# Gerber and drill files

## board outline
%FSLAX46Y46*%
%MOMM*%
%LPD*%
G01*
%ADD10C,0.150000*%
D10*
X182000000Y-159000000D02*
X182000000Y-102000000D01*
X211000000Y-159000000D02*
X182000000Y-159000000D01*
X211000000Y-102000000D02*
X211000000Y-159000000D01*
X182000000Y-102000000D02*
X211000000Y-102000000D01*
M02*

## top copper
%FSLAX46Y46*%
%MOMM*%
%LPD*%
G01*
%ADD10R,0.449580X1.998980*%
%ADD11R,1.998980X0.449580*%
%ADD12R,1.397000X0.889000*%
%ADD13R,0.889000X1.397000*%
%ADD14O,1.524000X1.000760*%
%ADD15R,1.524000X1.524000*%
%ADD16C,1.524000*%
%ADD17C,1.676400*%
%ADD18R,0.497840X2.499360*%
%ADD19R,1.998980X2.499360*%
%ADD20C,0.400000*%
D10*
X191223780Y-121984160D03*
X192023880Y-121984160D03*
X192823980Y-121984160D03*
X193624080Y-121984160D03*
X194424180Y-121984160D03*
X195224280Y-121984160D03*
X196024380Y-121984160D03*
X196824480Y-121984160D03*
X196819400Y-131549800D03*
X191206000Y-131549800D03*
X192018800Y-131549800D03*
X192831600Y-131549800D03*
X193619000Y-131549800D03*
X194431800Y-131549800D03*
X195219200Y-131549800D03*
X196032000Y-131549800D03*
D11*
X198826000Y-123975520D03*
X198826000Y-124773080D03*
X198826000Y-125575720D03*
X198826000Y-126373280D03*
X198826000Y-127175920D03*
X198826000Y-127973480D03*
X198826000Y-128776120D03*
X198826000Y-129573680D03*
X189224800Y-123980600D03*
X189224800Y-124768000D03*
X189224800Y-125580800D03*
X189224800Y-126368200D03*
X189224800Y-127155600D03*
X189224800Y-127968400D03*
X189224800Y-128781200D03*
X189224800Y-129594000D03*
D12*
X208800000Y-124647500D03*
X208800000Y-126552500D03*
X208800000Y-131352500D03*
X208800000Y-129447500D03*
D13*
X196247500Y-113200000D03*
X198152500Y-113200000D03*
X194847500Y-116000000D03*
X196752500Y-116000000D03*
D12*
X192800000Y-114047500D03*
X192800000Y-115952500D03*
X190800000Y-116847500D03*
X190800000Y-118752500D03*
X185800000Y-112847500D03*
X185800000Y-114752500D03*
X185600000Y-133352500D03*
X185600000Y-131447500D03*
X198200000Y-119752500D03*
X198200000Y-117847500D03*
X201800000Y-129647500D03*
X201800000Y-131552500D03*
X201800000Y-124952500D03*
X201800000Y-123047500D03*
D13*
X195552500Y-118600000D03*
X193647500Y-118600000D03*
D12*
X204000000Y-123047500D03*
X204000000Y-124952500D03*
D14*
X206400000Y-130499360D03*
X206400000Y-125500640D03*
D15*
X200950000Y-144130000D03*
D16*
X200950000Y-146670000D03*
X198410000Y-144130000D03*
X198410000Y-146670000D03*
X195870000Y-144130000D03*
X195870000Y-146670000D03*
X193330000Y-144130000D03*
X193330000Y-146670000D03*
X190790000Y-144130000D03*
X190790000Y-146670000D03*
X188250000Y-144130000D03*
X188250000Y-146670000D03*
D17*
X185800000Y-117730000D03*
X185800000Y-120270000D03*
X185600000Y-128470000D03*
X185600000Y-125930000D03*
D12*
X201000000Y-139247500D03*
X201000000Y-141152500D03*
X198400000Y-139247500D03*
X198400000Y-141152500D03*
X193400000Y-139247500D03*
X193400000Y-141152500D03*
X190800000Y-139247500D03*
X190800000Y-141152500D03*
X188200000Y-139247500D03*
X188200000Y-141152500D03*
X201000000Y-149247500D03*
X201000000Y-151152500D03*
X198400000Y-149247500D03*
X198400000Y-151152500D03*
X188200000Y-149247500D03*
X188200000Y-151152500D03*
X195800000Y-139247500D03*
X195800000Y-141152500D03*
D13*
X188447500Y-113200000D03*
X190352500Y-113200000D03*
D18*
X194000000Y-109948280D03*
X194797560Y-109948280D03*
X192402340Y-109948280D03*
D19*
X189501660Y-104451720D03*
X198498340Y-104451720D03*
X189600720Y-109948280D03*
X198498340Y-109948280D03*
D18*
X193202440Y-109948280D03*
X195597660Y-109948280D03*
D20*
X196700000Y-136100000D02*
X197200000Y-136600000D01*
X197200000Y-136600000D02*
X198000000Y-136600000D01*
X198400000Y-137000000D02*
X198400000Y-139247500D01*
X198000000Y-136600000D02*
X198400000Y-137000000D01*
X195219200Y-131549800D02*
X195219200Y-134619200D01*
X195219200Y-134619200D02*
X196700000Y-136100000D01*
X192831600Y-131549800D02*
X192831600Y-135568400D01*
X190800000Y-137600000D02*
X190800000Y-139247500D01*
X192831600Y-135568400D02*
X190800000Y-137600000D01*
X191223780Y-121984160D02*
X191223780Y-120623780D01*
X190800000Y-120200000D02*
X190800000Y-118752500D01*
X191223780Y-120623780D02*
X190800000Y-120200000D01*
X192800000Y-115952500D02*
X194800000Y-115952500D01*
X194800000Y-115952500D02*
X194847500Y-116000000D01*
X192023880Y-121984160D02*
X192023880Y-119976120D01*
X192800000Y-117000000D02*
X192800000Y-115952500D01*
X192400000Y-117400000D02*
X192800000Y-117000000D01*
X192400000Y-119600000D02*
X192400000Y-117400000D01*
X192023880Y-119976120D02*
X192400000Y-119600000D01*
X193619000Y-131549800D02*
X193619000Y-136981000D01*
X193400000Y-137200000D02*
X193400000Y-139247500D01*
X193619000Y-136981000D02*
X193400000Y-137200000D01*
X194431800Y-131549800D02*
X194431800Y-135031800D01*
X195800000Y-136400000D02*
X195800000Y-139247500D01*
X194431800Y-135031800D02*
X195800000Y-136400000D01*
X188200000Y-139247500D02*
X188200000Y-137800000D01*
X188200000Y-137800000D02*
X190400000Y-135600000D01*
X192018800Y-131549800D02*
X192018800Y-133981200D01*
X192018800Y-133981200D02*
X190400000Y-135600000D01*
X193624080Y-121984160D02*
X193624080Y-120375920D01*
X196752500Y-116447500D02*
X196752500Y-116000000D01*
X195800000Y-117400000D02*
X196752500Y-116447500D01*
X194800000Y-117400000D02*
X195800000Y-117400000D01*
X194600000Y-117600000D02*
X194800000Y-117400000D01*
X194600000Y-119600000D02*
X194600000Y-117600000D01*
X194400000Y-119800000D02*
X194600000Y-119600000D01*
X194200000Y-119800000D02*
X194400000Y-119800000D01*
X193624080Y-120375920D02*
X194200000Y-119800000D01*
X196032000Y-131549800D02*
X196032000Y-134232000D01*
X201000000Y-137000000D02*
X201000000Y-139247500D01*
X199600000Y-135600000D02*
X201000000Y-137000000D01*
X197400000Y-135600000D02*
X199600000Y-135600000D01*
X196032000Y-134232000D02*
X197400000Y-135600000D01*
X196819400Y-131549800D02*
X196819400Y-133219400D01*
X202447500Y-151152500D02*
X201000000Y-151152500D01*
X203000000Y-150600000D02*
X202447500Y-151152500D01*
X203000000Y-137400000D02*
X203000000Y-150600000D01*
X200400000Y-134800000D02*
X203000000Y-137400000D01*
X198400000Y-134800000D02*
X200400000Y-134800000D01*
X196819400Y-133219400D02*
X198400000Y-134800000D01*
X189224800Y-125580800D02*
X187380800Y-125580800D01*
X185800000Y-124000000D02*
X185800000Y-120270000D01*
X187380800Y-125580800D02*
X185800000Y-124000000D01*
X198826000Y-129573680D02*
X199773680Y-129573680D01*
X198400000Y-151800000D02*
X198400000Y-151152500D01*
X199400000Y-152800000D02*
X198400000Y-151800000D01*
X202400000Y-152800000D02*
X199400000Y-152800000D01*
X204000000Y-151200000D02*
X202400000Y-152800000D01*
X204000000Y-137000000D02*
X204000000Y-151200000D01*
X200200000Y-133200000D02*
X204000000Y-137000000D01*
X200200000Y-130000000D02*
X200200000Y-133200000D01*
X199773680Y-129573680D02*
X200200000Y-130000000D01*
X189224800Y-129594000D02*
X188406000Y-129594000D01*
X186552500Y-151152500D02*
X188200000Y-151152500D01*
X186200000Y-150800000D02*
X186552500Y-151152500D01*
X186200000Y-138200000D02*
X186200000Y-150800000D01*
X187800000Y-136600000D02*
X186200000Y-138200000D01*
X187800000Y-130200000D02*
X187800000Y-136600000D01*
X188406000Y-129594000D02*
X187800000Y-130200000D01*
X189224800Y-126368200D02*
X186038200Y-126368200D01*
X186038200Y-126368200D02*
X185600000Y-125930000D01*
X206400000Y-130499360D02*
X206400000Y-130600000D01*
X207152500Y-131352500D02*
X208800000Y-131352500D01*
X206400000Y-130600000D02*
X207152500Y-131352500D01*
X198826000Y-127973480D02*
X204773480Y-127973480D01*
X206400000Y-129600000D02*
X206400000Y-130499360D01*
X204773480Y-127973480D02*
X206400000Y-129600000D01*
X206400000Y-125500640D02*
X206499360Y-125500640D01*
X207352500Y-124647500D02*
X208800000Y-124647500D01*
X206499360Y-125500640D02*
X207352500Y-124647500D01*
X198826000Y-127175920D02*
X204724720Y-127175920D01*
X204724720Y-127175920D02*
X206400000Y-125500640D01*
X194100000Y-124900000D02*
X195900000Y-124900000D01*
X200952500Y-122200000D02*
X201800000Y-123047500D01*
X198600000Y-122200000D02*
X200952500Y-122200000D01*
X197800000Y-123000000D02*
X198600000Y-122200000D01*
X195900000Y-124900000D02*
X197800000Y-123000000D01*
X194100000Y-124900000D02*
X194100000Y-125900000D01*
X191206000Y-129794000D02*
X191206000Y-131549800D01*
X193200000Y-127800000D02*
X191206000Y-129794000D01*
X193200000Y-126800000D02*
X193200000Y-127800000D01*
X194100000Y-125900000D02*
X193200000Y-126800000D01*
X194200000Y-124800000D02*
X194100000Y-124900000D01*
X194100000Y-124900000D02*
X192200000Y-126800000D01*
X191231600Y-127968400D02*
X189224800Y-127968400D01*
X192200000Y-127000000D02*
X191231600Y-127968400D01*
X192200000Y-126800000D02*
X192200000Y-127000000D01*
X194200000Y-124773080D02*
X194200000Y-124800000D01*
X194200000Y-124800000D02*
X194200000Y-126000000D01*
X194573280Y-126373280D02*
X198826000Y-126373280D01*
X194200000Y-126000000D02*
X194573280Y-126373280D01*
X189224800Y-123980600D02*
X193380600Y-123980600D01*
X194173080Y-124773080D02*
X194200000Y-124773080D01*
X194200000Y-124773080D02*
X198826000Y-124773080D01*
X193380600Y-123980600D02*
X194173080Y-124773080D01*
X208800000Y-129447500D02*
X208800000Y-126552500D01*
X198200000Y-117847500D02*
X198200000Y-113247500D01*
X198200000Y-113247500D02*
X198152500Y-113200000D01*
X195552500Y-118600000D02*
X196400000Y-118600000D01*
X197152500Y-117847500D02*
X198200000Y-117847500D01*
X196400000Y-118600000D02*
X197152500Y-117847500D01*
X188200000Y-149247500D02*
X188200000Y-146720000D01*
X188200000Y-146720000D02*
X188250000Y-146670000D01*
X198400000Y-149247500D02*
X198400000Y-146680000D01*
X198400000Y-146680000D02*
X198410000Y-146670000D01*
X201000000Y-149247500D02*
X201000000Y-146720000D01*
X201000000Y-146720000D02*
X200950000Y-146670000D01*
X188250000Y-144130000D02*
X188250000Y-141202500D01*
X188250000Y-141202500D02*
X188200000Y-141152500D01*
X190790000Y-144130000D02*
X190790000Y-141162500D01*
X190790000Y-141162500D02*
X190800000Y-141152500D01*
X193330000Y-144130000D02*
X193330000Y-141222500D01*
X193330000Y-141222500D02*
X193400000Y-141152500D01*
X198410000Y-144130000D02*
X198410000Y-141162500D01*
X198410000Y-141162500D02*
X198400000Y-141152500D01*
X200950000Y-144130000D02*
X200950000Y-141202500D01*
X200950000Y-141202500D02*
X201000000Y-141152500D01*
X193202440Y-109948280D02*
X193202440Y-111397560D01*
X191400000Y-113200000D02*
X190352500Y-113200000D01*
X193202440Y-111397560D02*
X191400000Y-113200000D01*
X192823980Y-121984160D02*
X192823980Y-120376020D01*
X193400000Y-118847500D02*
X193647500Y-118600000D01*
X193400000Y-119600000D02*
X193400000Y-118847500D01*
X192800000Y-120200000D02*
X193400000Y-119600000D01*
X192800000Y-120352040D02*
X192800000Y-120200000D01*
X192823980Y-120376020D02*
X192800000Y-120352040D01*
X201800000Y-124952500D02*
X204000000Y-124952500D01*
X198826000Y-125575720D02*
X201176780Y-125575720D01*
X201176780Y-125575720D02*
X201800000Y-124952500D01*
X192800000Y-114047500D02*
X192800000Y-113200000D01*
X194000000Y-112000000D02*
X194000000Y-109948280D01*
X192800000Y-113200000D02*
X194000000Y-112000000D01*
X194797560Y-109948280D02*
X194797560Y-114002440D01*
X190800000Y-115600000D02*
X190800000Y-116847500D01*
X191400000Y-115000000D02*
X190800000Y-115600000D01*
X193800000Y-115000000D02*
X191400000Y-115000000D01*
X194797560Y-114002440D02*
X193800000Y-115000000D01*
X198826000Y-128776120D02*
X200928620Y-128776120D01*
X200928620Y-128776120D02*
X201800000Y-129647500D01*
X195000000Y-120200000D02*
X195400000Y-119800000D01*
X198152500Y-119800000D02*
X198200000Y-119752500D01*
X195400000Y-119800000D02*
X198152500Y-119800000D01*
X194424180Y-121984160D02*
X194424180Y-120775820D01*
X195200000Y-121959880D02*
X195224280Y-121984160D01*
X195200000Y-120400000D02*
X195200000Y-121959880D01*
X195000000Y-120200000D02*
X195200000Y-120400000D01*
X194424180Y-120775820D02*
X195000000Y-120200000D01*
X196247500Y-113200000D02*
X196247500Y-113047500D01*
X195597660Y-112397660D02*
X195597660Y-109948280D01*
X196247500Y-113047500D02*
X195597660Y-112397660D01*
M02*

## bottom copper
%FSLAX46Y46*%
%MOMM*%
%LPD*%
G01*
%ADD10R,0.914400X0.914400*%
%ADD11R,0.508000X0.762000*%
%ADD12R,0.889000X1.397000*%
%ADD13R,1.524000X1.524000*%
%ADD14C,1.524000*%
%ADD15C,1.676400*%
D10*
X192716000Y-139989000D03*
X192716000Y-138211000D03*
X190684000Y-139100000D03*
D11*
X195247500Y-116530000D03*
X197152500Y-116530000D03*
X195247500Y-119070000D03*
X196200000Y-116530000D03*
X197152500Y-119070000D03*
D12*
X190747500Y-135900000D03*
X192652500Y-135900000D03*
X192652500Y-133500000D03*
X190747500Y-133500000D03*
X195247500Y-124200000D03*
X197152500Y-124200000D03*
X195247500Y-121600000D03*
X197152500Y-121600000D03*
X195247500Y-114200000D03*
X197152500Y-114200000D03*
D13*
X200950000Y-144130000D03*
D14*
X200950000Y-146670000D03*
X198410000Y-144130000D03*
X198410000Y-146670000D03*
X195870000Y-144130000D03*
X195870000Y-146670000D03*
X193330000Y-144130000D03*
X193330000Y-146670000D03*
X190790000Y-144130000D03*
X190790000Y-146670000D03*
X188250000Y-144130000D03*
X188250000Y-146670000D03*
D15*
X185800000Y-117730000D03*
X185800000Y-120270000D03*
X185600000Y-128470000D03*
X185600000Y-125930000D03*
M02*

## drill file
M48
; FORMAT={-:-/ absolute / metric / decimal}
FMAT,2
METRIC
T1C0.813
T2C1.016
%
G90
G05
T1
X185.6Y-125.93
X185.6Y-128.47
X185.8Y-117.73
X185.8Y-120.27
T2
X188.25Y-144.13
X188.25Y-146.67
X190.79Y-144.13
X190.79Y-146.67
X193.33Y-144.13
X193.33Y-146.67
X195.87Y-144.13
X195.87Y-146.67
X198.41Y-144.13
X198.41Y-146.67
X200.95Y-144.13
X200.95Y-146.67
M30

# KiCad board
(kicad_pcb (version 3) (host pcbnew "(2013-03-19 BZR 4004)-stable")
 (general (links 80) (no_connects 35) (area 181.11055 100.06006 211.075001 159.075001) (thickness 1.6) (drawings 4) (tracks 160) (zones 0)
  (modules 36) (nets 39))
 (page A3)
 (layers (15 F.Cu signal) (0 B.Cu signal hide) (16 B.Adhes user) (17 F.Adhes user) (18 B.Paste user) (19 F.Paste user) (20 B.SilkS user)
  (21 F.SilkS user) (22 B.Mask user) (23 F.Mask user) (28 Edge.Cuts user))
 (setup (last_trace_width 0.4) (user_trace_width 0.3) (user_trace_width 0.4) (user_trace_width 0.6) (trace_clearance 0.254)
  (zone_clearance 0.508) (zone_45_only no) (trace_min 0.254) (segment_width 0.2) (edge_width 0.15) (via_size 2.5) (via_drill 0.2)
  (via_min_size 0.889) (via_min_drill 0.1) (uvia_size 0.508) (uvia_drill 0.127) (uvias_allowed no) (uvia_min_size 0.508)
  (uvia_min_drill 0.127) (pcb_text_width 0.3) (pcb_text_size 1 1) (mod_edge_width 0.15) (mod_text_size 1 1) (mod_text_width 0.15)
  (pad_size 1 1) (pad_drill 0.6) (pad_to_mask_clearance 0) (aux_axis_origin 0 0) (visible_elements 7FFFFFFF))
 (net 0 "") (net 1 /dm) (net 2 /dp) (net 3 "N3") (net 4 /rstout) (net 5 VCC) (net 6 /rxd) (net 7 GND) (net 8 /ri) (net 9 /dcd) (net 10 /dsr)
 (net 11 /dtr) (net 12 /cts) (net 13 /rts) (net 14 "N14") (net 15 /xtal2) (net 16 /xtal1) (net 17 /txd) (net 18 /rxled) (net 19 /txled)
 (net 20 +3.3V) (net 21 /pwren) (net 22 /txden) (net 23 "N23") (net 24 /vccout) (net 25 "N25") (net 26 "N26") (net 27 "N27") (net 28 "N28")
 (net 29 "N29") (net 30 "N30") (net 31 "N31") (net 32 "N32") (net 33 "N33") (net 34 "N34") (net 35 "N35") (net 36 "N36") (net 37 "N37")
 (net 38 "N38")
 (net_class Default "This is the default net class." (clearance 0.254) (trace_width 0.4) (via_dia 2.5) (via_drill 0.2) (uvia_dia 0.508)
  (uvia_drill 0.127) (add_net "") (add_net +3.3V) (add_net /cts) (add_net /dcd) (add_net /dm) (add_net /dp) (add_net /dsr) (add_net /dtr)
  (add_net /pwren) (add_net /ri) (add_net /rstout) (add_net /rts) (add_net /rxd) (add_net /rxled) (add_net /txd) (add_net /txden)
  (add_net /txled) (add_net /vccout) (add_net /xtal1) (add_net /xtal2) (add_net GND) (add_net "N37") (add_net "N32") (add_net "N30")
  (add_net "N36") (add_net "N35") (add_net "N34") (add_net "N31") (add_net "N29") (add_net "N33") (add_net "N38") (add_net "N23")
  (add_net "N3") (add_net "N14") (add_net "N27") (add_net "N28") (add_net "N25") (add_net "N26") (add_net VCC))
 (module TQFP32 (layer F.Cu) (at 194 126.8 270)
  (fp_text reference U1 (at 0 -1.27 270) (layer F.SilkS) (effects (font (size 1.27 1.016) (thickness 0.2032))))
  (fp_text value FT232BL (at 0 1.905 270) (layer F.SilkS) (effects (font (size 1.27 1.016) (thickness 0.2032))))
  (pad 8 smd rect (at -4.81584 2.77622 270) (size 1.99898 0.44958) (layers F.Cu F.Paste F.Mask) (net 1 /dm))
  (pad 7 smd rect (at -4.81584 1.97612 270) (size 1.99898 0.44958) (layers F.Cu F.Paste F.Mask) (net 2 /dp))
  (pad 6 smd rect (at -4.81584 1.17602 270) (size 1.99898 0.44958) (layers F.Cu F.Paste F.Mask) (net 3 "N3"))
  (pad 5 smd rect (at -4.81584 0.37592 270) (size 1.99898 0.44958) (layers F.Cu F.Paste F.Mask) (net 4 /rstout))
  (pad 4 smd rect (at -4.81584 -0.42418 270) (size 1.99898 0.44958) (layers F.Cu F.Paste F.Mask) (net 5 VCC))
  (pad 3 smd rect (at -4.81584 -1.22428 270) (size 1.99898 0.44958) (layers F.Cu F.Paste F.Mask) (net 5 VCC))
  (pad 2 smd rect (at -4.81584 -2.02438 270) (size 1.99898 0.44958) (layers F.Cu F.Paste F.Mask))
  (pad 1 smd rect (at -4.81584 -2.82448 270) (size 1.99898 0.44958) (layers F.Cu F.Paste F.Mask))
  (pad 24 smd rect (at 4.7498 -2.8194 270) (size 1.99898 0.44958) (layers F.Cu F.Paste F.Mask) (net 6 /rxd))
  (pad 17 smd rect (at 4.7498 2.794 270) (size 1.99898 0.44958) (layers F.Cu F.Paste F.Mask) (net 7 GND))
  (pad 18 smd rect (at 4.7498 1.9812 270) (size 1.99898 0.44958) (layers F.Cu F.Paste F.Mask) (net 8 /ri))
  (pad 19 smd rect (at 4.7498 1.1684 270) (size 1.99898 0.44958) (layers F.Cu F.Paste F.Mask) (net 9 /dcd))
  (pad 20 smd rect (at 4.7498 0.381 270) (size 1.99898 0.44958) (layers F.Cu F.Paste F.Mask) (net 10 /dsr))
  (pad 21 smd rect (at 4.7498 -0.4318 270) (size 1.99898 0.44958) (layers F.Cu F.Paste F.Mask) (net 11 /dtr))
  (pad 22 smd rect (at 4.7498 -1.2192 270) (size 1.99898 0.44958) (layers F.Cu F.Paste F.Mask) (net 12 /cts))
  (pad 23 smd rect (at 4.7498 -2.032 270) (size 1.99898 0.44958) (layers F.Cu F.Paste F.Mask) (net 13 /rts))
  (pad 32 smd rect (at -2.82448 -4.826 270) (size 0.44958 1.99898) (layers F.Cu F.Paste F.Mask))
  (pad 31 smd rect (at -2.02692 -4.826 270) (size 0.44958 1.99898) (layers F.Cu F.Paste F.Mask) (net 7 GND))
  (pad 30 smd rect (at -1.22428 -4.826 270) (size 0.44958 1.99898) (layers F.Cu F.Paste F.Mask) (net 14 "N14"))
  (pad 29 smd rect (at -0.42672 -4.826 270) (size 0.44958 1.99898) (layers F.Cu F.Paste F.Mask) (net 7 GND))
  (pad 28 smd rect (at 0.37592 -4.826 270) (size 0.44958 1.99898) (layers F.Cu F.Paste F.Mask) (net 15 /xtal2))
  (pad 27 smd rect (at 1.17348 -4.826 270) (size 0.44958 1.99898) (layers F.Cu F.Paste F.Mask) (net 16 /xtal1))
  (pad 26 smd rect (at 1.97612 -4.826 270) (size 0.44958 1.99898) (layers F.Cu F.Paste F.Mask) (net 5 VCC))
  (pad 25 smd rect (at 2.77368 -4.826 270) (size 0.44958 1.99898) (layers F.Cu F.Paste F.Mask) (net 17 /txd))
  (pad 9 smd rect (at -2.8194 4.7752 270) (size 0.44958 1.99898) (layers F.Cu F.Paste F.Mask) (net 7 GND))
  (pad 10 smd rect (at -2.032 4.7752 270) (size 0.44958 1.99898) (layers F.Cu F.Paste F.Mask))
  (pad 11 smd rect (at -1.2192 4.7752 270) (size 0.44958 1.99898) (layers F.Cu F.Paste F.Mask) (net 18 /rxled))
  (pad 12 smd rect (at -0.4318 4.7752 270) (size 0.44958 1.99898) (layers F.Cu F.Paste F.Mask) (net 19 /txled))
  (pad 13 smd rect (at 0.3556 4.7752 270) (size 0.44958 1.99898) (layers F.Cu F.Paste F.Mask) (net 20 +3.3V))
  (pad 14 smd rect (at 1.1684 4.7752 270) (size 0.44958 1.99898) (layers F.Cu F.Paste F.Mask) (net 7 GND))
  (pad 15 smd rect (at 1.9812 4.7752 270) (size 0.44958 1.99898) (layers F.Cu F.Paste F.Mask) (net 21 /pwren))
  (pad 16 smd rect (at 2.794 4.7752 270) (size 0.44958 1.99898) (layers F.Cu F.Paste F.Mask) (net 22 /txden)))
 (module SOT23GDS (layer B.Cu) (at 191.7 139.1 90)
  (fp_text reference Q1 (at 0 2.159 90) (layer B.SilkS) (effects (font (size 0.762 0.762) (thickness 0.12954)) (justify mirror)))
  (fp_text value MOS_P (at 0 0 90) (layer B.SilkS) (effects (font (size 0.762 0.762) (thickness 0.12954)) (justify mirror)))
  (pad S smd rect (at -0.889 1.016 90) (size 0.9144 0.9144) (layers B.Cu B.Paste B.Mask) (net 5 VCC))
  (pad G smd rect (at 0.889 1.016 90) (size 0.9144 0.9144) (layers B.Cu B.Paste B.Mask) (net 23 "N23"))
  (pad D smd rect (at 0 -1.016 90) (size 0.9144 0.9144) (layers B.Cu B.Paste B.Mask) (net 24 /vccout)))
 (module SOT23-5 (layer B.Cu) (at 196.2 117.8)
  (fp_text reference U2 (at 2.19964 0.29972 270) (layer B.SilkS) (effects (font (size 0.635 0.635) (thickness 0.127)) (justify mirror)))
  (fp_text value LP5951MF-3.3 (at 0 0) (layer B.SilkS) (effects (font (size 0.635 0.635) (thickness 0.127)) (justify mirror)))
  (pad 1 smd rect (at -0.9525 -1.27) (size 0.508 0.762) (layers B.Cu B.Paste B.Mask) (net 5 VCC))
  (pad 3 smd rect (at 0.9525 -1.27) (size 0.508 0.762) (layers B.Cu B.Paste B.Mask) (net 5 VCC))
  (pad 5 smd rect (at -0.9525 1.27) (size 0.508 0.762) (layers B.Cu B.Paste B.Mask) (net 20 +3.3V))
  (pad 2 smd rect (at 0 -1.27) (size 0.508 0.762) (layers B.Cu B.Paste B.Mask) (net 7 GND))
  (pad 4 smd rect (at 0.9525 1.27) (size 0.508 0.762) (layers B.Cu B.Paste B.Mask)))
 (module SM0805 (layer B.Cu) (at 191.7 135.9)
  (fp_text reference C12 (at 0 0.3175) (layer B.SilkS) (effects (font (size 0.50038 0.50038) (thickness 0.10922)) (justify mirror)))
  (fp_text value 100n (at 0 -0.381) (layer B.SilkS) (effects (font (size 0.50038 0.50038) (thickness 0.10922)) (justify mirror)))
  (pad 1 smd rect (at -0.9525 0) (size 0.889 1.397) (layers B.Cu B.Paste B.Mask) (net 24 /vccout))
  (pad 2 smd rect (at 0.9525 0) (size 0.889 1.397) (layers B.Cu B.Paste B.Mask) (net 23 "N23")))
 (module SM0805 (layer B.Cu) (at 191.7 133.5 180)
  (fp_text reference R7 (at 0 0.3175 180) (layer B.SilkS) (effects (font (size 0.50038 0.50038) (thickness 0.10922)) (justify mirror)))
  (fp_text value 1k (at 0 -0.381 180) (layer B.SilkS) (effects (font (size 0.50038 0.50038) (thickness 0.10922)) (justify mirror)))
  (pad 1 smd rect (at -0.9525 0 180) (size 0.889 1.397) (layers B.Cu B.Paste B.Mask) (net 23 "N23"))
  (pad 2 smd rect (at 0.9525 0 180) (size 0.889 1.397) (layers B.Cu B.Paste B.Mask) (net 21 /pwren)))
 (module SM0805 (layer F.Cu) (at 208.8 125.6 270)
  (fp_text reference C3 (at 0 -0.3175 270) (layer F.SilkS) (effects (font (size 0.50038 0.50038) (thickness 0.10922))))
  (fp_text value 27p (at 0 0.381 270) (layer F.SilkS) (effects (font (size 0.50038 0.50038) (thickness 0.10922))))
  (pad 1 smd rect (at -0.9525 0 270) (size 0.889 1.397) (layers F.Cu F.Paste F.Mask) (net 15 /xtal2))
  (pad 2 smd rect (at 0.9525 0 270) (size 0.889 1.397) (layers F.Cu F.Paste F.Mask) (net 7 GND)))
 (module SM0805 (layer F.Cu) (at 208.8 130.4 90)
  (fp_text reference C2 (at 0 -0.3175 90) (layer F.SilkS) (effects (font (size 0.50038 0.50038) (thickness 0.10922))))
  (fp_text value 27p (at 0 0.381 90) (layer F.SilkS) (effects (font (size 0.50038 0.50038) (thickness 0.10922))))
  (pad 1 smd rect (at -0.9525 0 90) (size 0.889 1.397) (layers F.Cu F.Paste F.Mask) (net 16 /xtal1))
  (pad 2 smd rect (at 0.9525 0 90) (size 0.889 1.397) (layers F.Cu F.Paste F.Mask) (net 7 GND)))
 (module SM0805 (layer B.Cu) (at 196.2 124.2)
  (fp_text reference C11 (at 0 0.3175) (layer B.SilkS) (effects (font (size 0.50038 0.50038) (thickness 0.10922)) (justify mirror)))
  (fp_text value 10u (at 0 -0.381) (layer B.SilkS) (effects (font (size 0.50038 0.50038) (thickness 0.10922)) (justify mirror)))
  (pad 1 smd rect (at -0.9525 0) (size 0.889 1.397) (layers B.Cu B.Paste B.Mask) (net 20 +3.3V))
  (pad 2 smd rect (at 0.9525 0) (size 0.889 1.397) (layers B.Cu B.Paste B.Mask) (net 7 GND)))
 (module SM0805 (layer B.Cu) (at 196.2 121.6)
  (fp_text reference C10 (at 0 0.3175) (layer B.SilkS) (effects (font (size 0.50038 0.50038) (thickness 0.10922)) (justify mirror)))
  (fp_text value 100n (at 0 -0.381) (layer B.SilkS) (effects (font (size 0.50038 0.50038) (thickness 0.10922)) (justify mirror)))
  (pad 1 smd rect (at -0.9525 0) (size 0.889 1.397) (layers B.Cu B.Paste B.Mask) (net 20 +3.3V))
  (pad 2 smd rect (at 0.9525 0) (size 0.889 1.397) (layers B.Cu B.Paste B.Mask) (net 7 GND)))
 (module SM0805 (layer B.Cu) (at 196.2 114.2)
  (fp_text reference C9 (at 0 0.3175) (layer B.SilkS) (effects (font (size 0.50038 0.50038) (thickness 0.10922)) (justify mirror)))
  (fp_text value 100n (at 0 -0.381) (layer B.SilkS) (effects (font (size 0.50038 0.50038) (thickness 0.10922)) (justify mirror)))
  (pad 1 smd rect (at -0.9525 0) (size 0.889 1.397) (layers B.Cu B.Paste B.Mask) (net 5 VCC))
  (pad 2 smd rect (at 0.9525 0) (size 0.889 1.397) (layers B.Cu B.Paste B.Mask) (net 7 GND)))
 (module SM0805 (layer F.Cu) (at 197.2 113.2)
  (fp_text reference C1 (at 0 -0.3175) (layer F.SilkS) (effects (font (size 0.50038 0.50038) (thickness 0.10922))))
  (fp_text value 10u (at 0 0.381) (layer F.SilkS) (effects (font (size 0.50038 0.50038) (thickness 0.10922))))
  (pad 1 smd rect (at -0.9525 0) (size 0.889 1.397) (layers F.Cu F.Paste F.Mask) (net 5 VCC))
  (pad 2 smd rect (at 0.9525 0) (size 0.889 1.397) (layers F.Cu F.Paste F.Mask) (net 7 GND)))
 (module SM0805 (layer F.Cu) (at 195.8 116)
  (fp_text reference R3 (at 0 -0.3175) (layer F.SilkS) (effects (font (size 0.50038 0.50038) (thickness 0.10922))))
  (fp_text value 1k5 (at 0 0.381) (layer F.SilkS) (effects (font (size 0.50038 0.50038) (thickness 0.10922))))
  (pad 1 smd rect (at -0.9525 0) (size 0.889 1.397) (layers F.Cu F.Paste F.Mask) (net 2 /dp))
  (pad 2 smd rect (at 0.9525 0) (size 0.889 1.397) (layers F.Cu F.Paste F.Mask) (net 4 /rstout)))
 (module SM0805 (layer F.Cu) (at 192.8 115 270)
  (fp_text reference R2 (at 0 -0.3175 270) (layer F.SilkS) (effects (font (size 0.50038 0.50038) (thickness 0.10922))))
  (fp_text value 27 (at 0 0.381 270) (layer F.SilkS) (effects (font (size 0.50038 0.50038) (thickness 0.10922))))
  (pad 1 smd rect (at -0.9525 0 270) (size 0.889 1.397) (layers F.Cu F.Paste F.Mask) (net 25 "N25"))
  (pad 2 smd rect (at 0.9525 0 270) (size 0.889 1.397) (layers F.Cu F.Paste F.Mask) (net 2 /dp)))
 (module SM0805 (layer F.Cu) (at 190.8 117.8 270)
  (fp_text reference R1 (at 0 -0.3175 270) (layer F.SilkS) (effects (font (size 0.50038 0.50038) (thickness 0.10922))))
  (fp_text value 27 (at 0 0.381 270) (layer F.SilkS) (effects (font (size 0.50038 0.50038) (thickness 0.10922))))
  (pad 1 smd rect (at -0.9525 0 270) (size 0.889 1.397) (layers F.Cu F.Paste F.Mask) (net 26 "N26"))
  (pad 2 smd rect (at 0.9525 0 270) (size 0.889 1.397) (layers F.Cu F.Paste F.Mask) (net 1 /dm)))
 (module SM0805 (layer F.Cu) (at 185.8 113.8 270)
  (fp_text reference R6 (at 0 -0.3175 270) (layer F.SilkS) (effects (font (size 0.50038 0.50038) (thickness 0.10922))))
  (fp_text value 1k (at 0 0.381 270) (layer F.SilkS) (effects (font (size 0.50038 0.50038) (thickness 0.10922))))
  (pad 1 smd rect (at -0.9525 0 270) (size 0.889 1.397) (layers F.Cu F.Paste F.Mask) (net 5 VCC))
  (pad 2 smd rect (at 0.9525 0 270) (size 0.889 1.397) (layers F.Cu F.Paste F.Mask) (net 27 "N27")))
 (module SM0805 (layer F.Cu) (at 185.6 132.4 90)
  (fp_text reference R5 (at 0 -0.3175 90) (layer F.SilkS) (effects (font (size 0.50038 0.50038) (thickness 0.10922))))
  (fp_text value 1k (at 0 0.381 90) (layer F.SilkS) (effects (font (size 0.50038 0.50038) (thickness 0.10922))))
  (pad 1 smd rect (at -0.9525 0 90) (size 0.889 1.397) (layers F.Cu F.Paste F.Mask) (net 5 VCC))
  (pad 2 smd rect (at 0.9525 0 90) (size 0.889 1.397) (layers F.Cu F.Paste F.Mask) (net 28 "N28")))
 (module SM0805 (layer F.Cu) (at 198.2 118.8 90)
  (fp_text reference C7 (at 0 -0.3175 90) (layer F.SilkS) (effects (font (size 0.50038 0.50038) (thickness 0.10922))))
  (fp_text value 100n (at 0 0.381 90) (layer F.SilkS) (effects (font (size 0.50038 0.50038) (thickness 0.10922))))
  (pad 1 smd rect (at -0.9525 0 90) (size 0.889 1.397) (layers F.Cu F.Paste F.Mask) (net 5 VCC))
  (pad 2 smd rect (at 0.9525 0 90) (size 0.889 1.397) (layers F.Cu F.Paste F.Mask) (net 7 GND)))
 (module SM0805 (layer F.Cu) (at 201.8 130.6 270)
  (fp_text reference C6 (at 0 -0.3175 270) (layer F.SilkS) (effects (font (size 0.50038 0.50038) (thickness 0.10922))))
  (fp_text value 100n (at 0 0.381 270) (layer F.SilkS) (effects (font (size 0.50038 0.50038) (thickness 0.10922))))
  (pad 1 smd rect (at -0.9525 0 270) (size 0.889 1.397) (layers F.Cu F.Paste F.Mask) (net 5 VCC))
  (pad 2 smd rect (at 0.9525 0 270) (size 0.889 1.397) (layers F.Cu F.Paste F.Mask) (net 7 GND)))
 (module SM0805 (layer F.Cu) (at 201.8 124 90)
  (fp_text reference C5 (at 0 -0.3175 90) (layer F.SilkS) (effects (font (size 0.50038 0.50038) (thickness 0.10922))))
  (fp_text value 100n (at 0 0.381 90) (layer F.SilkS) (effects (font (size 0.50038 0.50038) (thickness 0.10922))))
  (pad 1 smd rect (at -0.9525 0 90) (size 0.889 1.397) (layers F.Cu F.Paste F.Mask) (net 14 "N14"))
  (pad 2 smd rect (at 0.9525 0 90) (size 0.889 1.397) (layers F.Cu F.Paste F.Mask) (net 7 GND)))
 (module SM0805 (layer F.Cu) (at 194.6 118.6 180)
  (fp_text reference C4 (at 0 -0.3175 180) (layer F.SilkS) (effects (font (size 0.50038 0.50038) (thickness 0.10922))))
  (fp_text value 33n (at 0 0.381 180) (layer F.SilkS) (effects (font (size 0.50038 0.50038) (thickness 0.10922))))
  (pad 1 smd rect (at -0.9525 0 180) (size 0.889 1.397) (layers F.Cu F.Paste F.Mask) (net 7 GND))
  (pad 2 smd rect (at 0.9525 0 180) (size 0.889 1.397) (layers F.Cu F.Paste F.Mask) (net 3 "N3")))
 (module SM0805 (layer F.Cu) (at 204 124 270)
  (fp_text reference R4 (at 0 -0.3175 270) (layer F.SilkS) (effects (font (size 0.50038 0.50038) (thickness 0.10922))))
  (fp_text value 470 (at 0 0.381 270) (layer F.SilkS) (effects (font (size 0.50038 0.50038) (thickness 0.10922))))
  (pad 1 smd rect (at -0.9525 0 270) (size 0.889 1.397) (layers F.Cu F.Paste F.Mask) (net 5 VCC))
  (pad 2 smd rect (at 0.9525 0 270) (size 0.889 1.397) (layers F.Cu F.Paste F.Mask) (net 14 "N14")))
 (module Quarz (layer F.Cu) (at 206.4 128 90)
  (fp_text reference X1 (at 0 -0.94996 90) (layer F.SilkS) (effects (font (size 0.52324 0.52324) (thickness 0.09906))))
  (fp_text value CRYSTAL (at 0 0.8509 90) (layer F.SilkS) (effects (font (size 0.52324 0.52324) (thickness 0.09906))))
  (pad 1 smd oval (at -2.49936 0 90) (size 1.00076 1.524) (layers F.Cu F.Paste F.Mask) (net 16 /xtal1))
  (pad 2 smd oval (at 2.49936 0 90) (size 1.00076 1.524) (layers F.Cu F.Paste F.Mask) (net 15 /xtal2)))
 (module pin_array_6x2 (layer F.Cu) (at 194.6 145.4 180)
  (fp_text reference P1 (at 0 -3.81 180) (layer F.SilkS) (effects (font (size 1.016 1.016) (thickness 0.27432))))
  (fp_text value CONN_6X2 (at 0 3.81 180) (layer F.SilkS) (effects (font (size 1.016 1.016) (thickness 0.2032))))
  (pad 1 thru_hole rect (at -6.35 1.27 180) (size 1.524 1.524) (drill 1.016) (layers *.Cu *.Mask F.SilkS) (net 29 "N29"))
  (pad 2 thru_hole circle (at -6.35 -1.27 180) (size 1.524 1.524) (drill 1.016) (layers *.Cu *.Mask F.SilkS) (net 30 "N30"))
  (pad 3 thru_hole circle (at -3.81 1.27 180) (size 1.524 1.524) (drill 1.016) (layers *.Cu *.Mask F.SilkS) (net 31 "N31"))
  (pad 4 thru_hole circle (at -3.81 -1.27 180) (size 1.524 1.524) (drill 1.016) (layers *.Cu *.Mask F.SilkS) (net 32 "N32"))
  (pad 5 thru_hole circle (at -1.27 1.27 180) (size 1.524 1.524) (drill 1.016) (layers *.Cu *.Mask F.SilkS) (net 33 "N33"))
  (pad 6 thru_hole circle (at -1.27 -1.27 180) (size 1.524 1.524) (drill 1.016) (layers *.Cu *.Mask F.SilkS) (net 7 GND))
  (pad 7 thru_hole circle (at 1.27 1.27 180) (size 1.524 1.524) (drill 1.016) (layers *.Cu *.Mask F.SilkS) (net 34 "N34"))
  (pad 8 thru_hole circle (at 1.27 -1.27 180) (size 1.524 1.524) (drill 1.016) (layers *.Cu *.Mask F.SilkS) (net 24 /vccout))
  (pad 9 thru_hole circle (at 3.81 1.27 180) (size 1.524 1.524) (drill 1.016) (layers *.Cu *.Mask F.SilkS) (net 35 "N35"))
  (pad 10 thru_hole circle (at 3.81 -1.27 180) (size 1.524 1.524) (drill 1.016) (layers *.Cu *.Mask F.SilkS) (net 20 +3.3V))
  (pad 11 thru_hole circle (at 6.35 1.27 180) (size 1.524 1.524) (drill 1.016) (layers *.Cu *.Mask F.SilkS) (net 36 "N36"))
  (pad 12 thru_hole circle (at 6.35 -1.27 180) (size 1.524 1.524) (drill 1.016) (layers *.Cu *.Mask F.SilkS) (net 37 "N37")))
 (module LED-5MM (layer F.Cu) (at 185.8 119 270)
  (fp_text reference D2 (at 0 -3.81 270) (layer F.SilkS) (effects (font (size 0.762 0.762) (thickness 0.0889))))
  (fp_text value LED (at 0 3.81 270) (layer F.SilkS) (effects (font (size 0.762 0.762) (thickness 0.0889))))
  (pad 1 thru_hole circle (at -1.27 0 270) (size 1.6764 1.6764) (drill 0.812799) (layers *.Cu *.Mask F.SilkS) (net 27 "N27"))
  (pad 2 thru_hole circle (at 1.27 0 270) (size 1.6764 1.6764) (drill 0.812799) (layers *.Cu *.Mask F.SilkS) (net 18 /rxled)))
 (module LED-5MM (layer F.Cu) (at 185.6 127.2 90)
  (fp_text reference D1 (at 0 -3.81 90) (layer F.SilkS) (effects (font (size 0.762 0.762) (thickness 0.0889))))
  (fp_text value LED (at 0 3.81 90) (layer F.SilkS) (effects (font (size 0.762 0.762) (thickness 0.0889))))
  (pad 1 thru_hole circle (at -1.27 0 90) (size 1.6764 1.6764) (drill 0.812799) (layers *.Cu *.Mask F.SilkS) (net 28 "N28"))
  (pad 2 thru_hole circle (at 1.27 0 90) (size 1.6764 1.6764) (drill 0.812799) (layers *.Cu *.Mask F.SilkS) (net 19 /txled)))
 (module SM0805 (layer F.Cu) (at 201 140.2 270)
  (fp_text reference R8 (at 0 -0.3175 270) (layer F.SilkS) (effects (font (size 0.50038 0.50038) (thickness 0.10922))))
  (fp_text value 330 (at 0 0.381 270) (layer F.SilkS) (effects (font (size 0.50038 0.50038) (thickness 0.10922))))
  (pad 1 smd rect (at -0.9525 0 270) (size 0.889 1.397) (layers F.Cu F.Paste F.Mask) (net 13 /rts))
  (pad 2 smd rect (at 0.9525 0 270) (size 0.889 1.397) (layers F.Cu F.Paste F.Mask) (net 29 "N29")))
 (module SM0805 (layer F.Cu) (at 198.4 140.2 270)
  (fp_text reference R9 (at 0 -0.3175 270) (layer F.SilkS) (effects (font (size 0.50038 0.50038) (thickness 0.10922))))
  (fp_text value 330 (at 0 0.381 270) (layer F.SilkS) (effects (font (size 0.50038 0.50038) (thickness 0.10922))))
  (pad 1 smd rect (at -0.9525 0 270) (size 0.889 1.397) (layers F.Cu F.Paste F.Mask) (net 12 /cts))
  (pad 2 smd rect (at 0.9525 0 270) (size 0.889 1.397) (layers F.Cu F.Paste F.Mask) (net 31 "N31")))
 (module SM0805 (layer F.Cu) (at 193.4 140.2 270)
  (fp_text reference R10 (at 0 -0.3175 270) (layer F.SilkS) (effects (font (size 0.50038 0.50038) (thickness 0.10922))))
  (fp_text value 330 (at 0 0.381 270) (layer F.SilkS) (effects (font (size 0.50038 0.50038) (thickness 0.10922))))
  (pad 1 smd rect (at -0.9525 0 270) (size 0.889 1.397) (layers F.Cu F.Paste F.Mask) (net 10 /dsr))
  (pad 2 smd rect (at 0.9525 0 270) (size 0.889 1.397) (layers F.Cu F.Paste F.Mask) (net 34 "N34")))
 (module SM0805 (layer F.Cu) (at 190.8 140.2 270)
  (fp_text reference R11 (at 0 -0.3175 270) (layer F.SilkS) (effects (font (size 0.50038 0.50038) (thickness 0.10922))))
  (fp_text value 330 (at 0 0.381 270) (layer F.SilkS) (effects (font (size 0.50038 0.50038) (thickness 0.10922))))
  (pad 1 smd rect (at -0.9525 0 270) (size 0.889 1.397) (layers F.Cu F.Paste F.Mask) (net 9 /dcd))
  (pad 2 smd rect (at 0.9525 0 270) (size 0.889 1.397) (layers F.Cu F.Paste F.Mask) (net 35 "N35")))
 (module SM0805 (layer F.Cu) (at 188.2 140.2 270)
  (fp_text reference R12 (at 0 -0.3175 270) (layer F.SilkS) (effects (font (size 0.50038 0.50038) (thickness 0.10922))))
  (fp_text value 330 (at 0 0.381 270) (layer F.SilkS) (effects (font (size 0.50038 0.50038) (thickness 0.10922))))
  (pad 1 smd rect (at -0.9525 0 270) (size 0.889 1.397) (layers F.Cu F.Paste F.Mask) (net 8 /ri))
  (pad 2 smd rect (at 0.9525 0 270) (size 0.889 1.397) (layers F.Cu F.Paste F.Mask) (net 36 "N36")))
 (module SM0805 (layer F.Cu) (at 201 150.2 270)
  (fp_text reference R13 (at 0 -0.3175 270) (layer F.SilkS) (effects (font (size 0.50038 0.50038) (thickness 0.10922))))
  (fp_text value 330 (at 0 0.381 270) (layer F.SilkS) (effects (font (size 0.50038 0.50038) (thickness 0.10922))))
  (pad 1 smd rect (at -0.9525 0 270) (size 0.889 1.397) (layers F.Cu F.Paste F.Mask) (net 30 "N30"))
  (pad 2 smd rect (at 0.9525 0 270) (size 0.889 1.397) (layers F.Cu F.Paste F.Mask) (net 6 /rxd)))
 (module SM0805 (layer F.Cu) (at 198.4 150.2 270)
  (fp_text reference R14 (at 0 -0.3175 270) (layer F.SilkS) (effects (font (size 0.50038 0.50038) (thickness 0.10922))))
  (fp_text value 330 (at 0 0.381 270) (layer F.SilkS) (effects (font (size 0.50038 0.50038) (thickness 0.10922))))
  (pad 1 smd rect (at -0.9525 0 270) (size 0.889 1.397) (layers F.Cu F.Paste F.Mask) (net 32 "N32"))
  (pad 2 smd rect (at 0.9525 0 270) (size 0.889 1.397) (layers F.Cu F.Paste F.Mask) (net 17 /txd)))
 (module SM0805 (layer F.Cu) (at 188.2 150.2 270)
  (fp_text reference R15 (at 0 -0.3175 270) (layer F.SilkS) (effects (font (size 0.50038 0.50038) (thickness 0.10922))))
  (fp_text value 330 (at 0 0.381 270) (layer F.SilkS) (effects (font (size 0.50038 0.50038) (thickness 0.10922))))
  (pad 1 smd rect (at -0.9525 0 270) (size 0.889 1.397) (layers F.Cu F.Paste F.Mask) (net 37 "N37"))
  (pad 2 smd rect (at 0.9525 0 270) (size 0.889 1.397) (layers F.Cu F.Paste F.Mask) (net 22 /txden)))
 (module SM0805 (layer F.Cu) (at 195.8 140.2 270)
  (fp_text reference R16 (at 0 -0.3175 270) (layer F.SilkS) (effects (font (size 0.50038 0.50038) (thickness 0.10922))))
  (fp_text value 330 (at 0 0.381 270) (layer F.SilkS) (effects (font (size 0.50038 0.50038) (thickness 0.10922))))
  (pad 1 smd rect (at -0.9525 0 270) (size 0.889 1.397) (layers F.Cu F.Paste F.Mask) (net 11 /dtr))
  (pad 2 smd rect (at 0.9525 0 270) (size 0.889 1.397) (layers F.Cu F.Paste F.Mask) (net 33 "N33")))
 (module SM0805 (layer F.Cu) (at 189.4 113.2)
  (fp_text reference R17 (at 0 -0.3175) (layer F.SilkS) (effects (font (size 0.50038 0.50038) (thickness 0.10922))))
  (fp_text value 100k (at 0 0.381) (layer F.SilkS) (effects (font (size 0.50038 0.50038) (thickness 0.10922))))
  (pad 1 smd rect (at -0.9525 0) (size 0.889 1.397) (layers F.Cu F.Paste F.Mask) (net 7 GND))
  (pad 2 smd rect (at 0.9525 0) (size 0.889 1.397) (layers F.Cu F.Paste F.Mask) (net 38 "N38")))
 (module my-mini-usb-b (layer F.Cu) (at 194 107.2 270)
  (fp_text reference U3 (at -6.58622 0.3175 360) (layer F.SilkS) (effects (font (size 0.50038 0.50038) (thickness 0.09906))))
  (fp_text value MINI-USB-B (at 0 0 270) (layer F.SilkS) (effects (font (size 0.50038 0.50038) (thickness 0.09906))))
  (pad 3 smd rect (at 2.74828 0 270) (size 2.49936 0.49784) (layers F.Cu F.Paste F.Mask) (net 25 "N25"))
  (pad 2 smd rect (at 2.74828 -0.79756 270) (size 2.49936 0.49784) (layers F.Cu F.Paste F.Mask) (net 26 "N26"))
  (pad 5 smd rect (at 2.74828 1.59766 270) (size 2.49936 0.49784) (layers F.Cu F.Paste F.Mask) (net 7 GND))
  (pad 0 smd rect (at -2.74828 4.49834 270) (size 2.49936 1.99898) (layers F.Cu F.Paste F.Mask) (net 7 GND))
  (pad 0 smd rect (at -2.74828 -4.49834 270) (size 2.49936 1.99898) (layers F.Cu F.Paste F.Mask) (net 7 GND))
  (pad 0 smd rect (at 2.74828 4.39928 270) (size 2.49936 1.99898) (layers F.Cu F.Paste F.Mask) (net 7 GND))
  (pad 0 smd rect (at 2.74828 -4.49834 270) (size 2.49936 1.99898) (layers F.Cu F.Paste F.Mask) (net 7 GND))
  (pad 4 smd rect (at 2.74828 0.79756 270) (size 2.49936 0.49784) (layers F.Cu F.Paste F.Mask) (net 38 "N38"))
  (pad 1 smd rect (at 2.74828 -1.59766 270) (size 2.49936 0.49784) (layers F.Cu F.Paste F.Mask) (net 5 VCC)))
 (gr_line (start 182 159) (end 182 102) (angle 90) (layer Edge.Cuts) (width 0.15))
 (gr_line (start 211 159) (end 182 159) (angle 90) (layer Edge.Cuts) (width 0.15))
 (gr_line (start 211 102) (end 211 159) (angle 90) (layer Edge.Cuts) (width 0.15))
 (gr_line (start 182 102) (end 211 102) (angle 90) (layer Edge.Cuts) (width 0.15))
 (segment (start 196.7 136.1) (end 197.2 136.6) (width 0.4) (layer F.Cu) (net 12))
 (segment (start 197.2 136.6) (end 198 136.6) (width 0.4) (layer F.Cu) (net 12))
 (segment (start 198.4 137) (end 198.4 139.2475) (width 0.4) (layer F.Cu) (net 12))
 (segment (start 198 136.6) (end 198.4 137) (width 0.4) (layer F.Cu) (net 12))
 (segment (start 195.2192 131.5498) (end 195.2192 134.6192) (width 0.4) (layer F.Cu) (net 12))
 (segment (start 195.2192 134.6192) (end 196.7 136.1) (width 0.4) (layer F.Cu) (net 12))
 (segment (start 192.8316 131.5498) (end 192.8316 135.5684) (width 0.4) (layer F.Cu) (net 9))
 (segment (start 190.8 137.6) (end 190.8 139.2475) (width 0.4) (layer F.Cu) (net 9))
 (segment (start 192.8316 135.5684) (end 190.8 137.6) (width 0.4) (layer F.Cu) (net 9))
 (segment (start 191.22378 121.98416) (end 191.22378 120.62378) (width 0.4) (layer F.Cu) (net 1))
 (segment (start 190.8 120.2) (end 190.8 118.7525) (width 0.4) (layer F.Cu) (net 1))
 (segment (start 191.22378 120.62378) (end 190.8 120.2) (width 0.4) (layer F.Cu) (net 1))
 (segment (start 192.8 115.9525) (end 194.8 115.9525) (width 0.4) (layer F.Cu) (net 2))
 (segment (start 194.8 115.9525) (end 194.8475 116) (width 0.4) (layer F.Cu) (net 2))
 (segment (start 192.02388 121.98416) (end 192.02388 119.97612) (width 0.4) (layer F.Cu) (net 2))
 (segment (start 192.8 117) (end 192.8 115.9525) (width 0.4) (layer F.Cu) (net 2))
 (segment (start 192.4 117.4) (end 192.8 117) (width 0.4) (layer F.Cu) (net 2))
 (segment (start 192.4 119.6) (end 192.4 117.4) (width 0.4) (layer F.Cu) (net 2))
 (segment (start 192.02388 119.97612) (end 192.4 119.6) (width 0.4) (layer F.Cu) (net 2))
 (segment (start 193.619 131.5498) (end 193.619 136.981) (width 0.4) (layer F.Cu) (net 10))
 (segment (start 193.4 137.2) (end 193.4 139.2475) (width 0.4) (layer F.Cu) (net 10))
 (segment (start 193.619 136.981) (end 193.4 137.2) (width 0.4) (layer F.Cu) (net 10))
 (segment (start 194.4318 131.5498) (end 194.4318 135.0318) (width 0.4) (layer F.Cu) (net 11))
 (segment (start 195.8 136.4) (end 195.8 139.2475) (width 0.4) (layer F.Cu) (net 11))
 (segment (start 194.4318 135.0318) (end 195.8 136.4) (width 0.4) (layer F.Cu) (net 11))
 (segment (start 188.2 139.2475) (end 188.2 137.8) (width 0.4) (layer F.Cu) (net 8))
 (segment (start 188.2 137.8) (end 190.4 135.6) (width 0.4) (layer F.Cu) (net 8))
 (segment (start 192.0188 131.5498) (end 192.0188 133.9812) (width 0.4) (layer F.Cu) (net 8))
 (segment (start 192.0188 133.9812) (end 190.4 135.6) (width 0.4) (layer F.Cu) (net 8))
 (segment (start 193.62408 121.98416) (end 193.62408 120.37592) (width 0.4) (layer F.Cu) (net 4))
 (segment (start 196.7525 116.4475) (end 196.7525 116) (width 0.4) (layer F.Cu) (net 4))
 (segment (start 195.8 117.4) (end 196.7525 116.4475) (width 0.4) (layer F.Cu) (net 4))
 (segment (start 194.8 117.4) (end 195.8 117.4) (width 0.4) (layer F.Cu) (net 4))
 (segment (start 194.6 117.6) (end 194.8 117.4) (width 0.4) (layer F.Cu) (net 4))
 (segment (start 194.6 119.6) (end 194.6 117.6) (width 0.4) (layer F.Cu) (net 4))
 (segment (start 194.4 119.8) (end 194.6 119.6) (width 0.4) (layer F.Cu) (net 4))
 (segment (start 194.2 119.8) (end 194.4 119.8) (width 0.4) (layer F.Cu) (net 4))
 (segment (start 193.62408 120.37592) (end 194.2 119.8) (width 0.4) (layer F.Cu) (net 4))
 (segment (start 196.032 131.5498) (end 196.032 134.232) (width 0.4) (layer F.Cu) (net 13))
 (segment (start 201 137) (end 201 139.2475) (width 0.4) (layer F.Cu) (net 13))
 (segment (start 199.6 135.6) (end 201 137) (width 0.4) (layer F.Cu) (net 13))
 (segment (start 197.4 135.6) (end 199.6 135.6) (width 0.4) (layer F.Cu) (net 13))
 (segment (start 196.032 134.232) (end 197.4 135.6) (width 0.4) (layer F.Cu) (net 13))
 (segment (start 196.8194 131.5498) (end 196.8194 133.2194) (width 0.4) (layer F.Cu) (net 6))
 (segment (start 202.4475 151.1525) (end 201 151.1525) (width 0.4) (layer F.Cu) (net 6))
 (segment (start 203 150.6) (end 202.4475 151.1525) (width 0.4) (layer F.Cu) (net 6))
 (segment (start 203 137.4) (end 203 150.6) (width 0.4) (layer F.Cu) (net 6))
 (segment (start 200.4 134.8) (end 203 137.4) (width 0.4) (layer F.Cu) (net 6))
 (segment (start 198.4 134.8) (end 200.4 134.8) (width 0.4) (layer F.Cu) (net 6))
 (segment (start 196.8194 133.2194) (end 198.4 134.8) (width 0.4) (layer F.Cu) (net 6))
 (segment (start 189.2248 125.5808) (end 187.3808 125.5808) (width 0.4) (layer F.Cu) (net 18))
 (segment (start 185.8 124) (end 185.8 120.27) (width 0.4) (layer F.Cu) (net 18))
 (segment (start 187.3808 125.5808) (end 185.8 124) (width 0.4) (layer F.Cu) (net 18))
 (segment (start 198.826 129.57368) (end 199.77368 129.57368) (width 0.4) (layer F.Cu) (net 17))
 (segment (start 198.4 151.8) (end 198.4 151.1525) (width 0.4) (layer F.Cu) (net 17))
 (segment (start 199.4 152.8) (end 198.4 151.8) (width 0.4) (layer F.Cu) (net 17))
 (segment (start 202.4 152.8) (end 199.4 152.8) (width 0.4) (layer F.Cu) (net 17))
 (segment (start 204 151.2) (end 202.4 152.8) (width 0.4) (layer F.Cu) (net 17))
 (segment (start 204 137) (end 204 151.2) (width 0.4) (layer F.Cu) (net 17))
 (segment (start 200.2 133.2) (end 204 137) (width 0.4) (layer F.Cu) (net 17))
 (segment (start 200.2 130) (end 200.2 133.2) (width 0.4) (layer F.Cu) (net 17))
 (segment (start 199.77368 129.57368) (end 200.2 130) (width 0.4) (layer F.Cu) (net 17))
 (segment (start 189.2248 129.594) (end 188.406 129.594) (width 0.4) (layer F.Cu) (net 22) (status C00000))
 (segment (start 186.5525 151.1525) (end 188.2 151.1525) (width 0.4) (layer F.Cu) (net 22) (status 800000))
 (segment (start 186.2 150.8) (end 186.5525 151.1525) (width 0.4) (layer F.Cu) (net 22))
 (segment (start 186.2 138.2) (end 186.2 150.8) (width 0.4) (layer F.Cu) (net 22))
 (segment (start 187.8 136.6) (end 186.2 138.2) (width 0.4) (layer F.Cu) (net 22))
 (segment (start 187.8 130.2) (end 187.8 136.6) (width 0.4) (layer F.Cu) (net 22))
 (segment (start 188.406 129.594) (end 187.8 130.2) (width 0.4) (layer F.Cu) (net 22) (status 400000))
 (segment (start 189.2248 126.3682) (end 186.0382 126.3682) (width 0.4) (layer F.Cu) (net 19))
 (segment (start 186.0382 126.3682) (end 185.6 125.93) (width 0.4) (layer F.Cu) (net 19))
 (segment (start 206.4 130.49936) (end 206.4 130.6) (width 0.4) (layer F.Cu) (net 16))
 (segment (start 207.1525 131.3525) (end 208.8 131.3525) (width 0.4) (layer F.Cu) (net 16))
 (segment (start 206.4 130.6) (end 207.1525 131.3525) (width 0.4) (layer F.Cu) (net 16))
 (segment (start 198.826 127.97348) (end 204.77348 127.97348) (width 0.4) (layer F.Cu) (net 16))
 (segment (start 206.4 129.6) (end 206.4 130.49936) (width 0.4) (layer F.Cu) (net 16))
 (segment (start 204.77348 127.97348) (end 206.4 129.6) (width 0.4) (layer F.Cu) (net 16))
 (segment (start 206.4 125.50064) (end 206.49936 125.50064) (width 0.4) (layer F.Cu) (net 15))
 (segment (start 207.3525 124.6475) (end 208.8 124.6475) (width 0.4) (layer F.Cu) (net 15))
 (segment (start 206.49936 125.50064) (end 207.3525 124.6475) (width 0.4) (layer F.Cu) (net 15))
 (segment (start 198.826 127.17592) (end 204.72472 127.17592) (width 0.4) (layer F.Cu) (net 15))
 (segment (start 204.72472 127.17592) (end 206.4 125.50064) (width 0.4) (layer F.Cu) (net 15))
 (segment (start 194.1 124.9) (end 195.9 124.9) (width 0.4) (layer F.Cu) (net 7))
 (segment (start 200.9525 122.2) (end 201.8 123.0475) (width 0.4) (layer F.Cu) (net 7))
 (segment (start 198.6 122.2) (end 200.9525 122.2) (width 0.4) (layer F.Cu) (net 7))
 (segment (start 197.8 123) (end 198.6 122.2) (width 0.4) (layer F.Cu) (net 7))
 (segment (start 195.9 124.9) (end 197.8 123) (width 0.4) (layer F.Cu) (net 7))
 (segment (start 194.1 124.9) (end 194.1 125.9) (width 0.4) (layer F.Cu) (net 7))
 (segment (start 191.206 129.794) (end 191.206 131.5498) (width 0.4) (layer F.Cu) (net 7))
 (segment (start 193.2 127.8) (end 191.206 129.794) (width 0.4) (layer F.Cu) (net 7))
 (segment (start 193.2 126.8) (end 193.2 127.8) (width 0.4) (layer F.Cu) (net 7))
 (segment (start 194.1 125.9) (end 193.2 126.8) (width 0.4) (layer F.Cu) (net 7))
 (segment (start 194.2 124.8) (end 194.1 124.9) (width 0.4) (layer F.Cu) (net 7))
 (segment (start 194.1 124.9) (end 192.2 126.8) (width 0.4) (layer F.Cu) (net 7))
 (segment (start 191.2316 127.9684) (end 189.2248 127.9684) (width 0.4) (layer F.Cu) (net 7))
 (segment (start 192.2 127) (end 191.2316 127.9684) (width 0.4) (layer F.Cu) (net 7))
 (segment (start 192.2 126.8) (end 192.2 127) (width 0.4) (layer F.Cu) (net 7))
 (segment (start 194.2 124.77308) (end 194.2 124.8) (width 0.4) (layer F.Cu) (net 7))
 (segment (start 194.2 124.8) (end 194.2 126) (width 0.4) (layer F.Cu) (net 7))
 (segment (start 194.57328 126.37328) (end 198.826 126.37328) (width 0.4) (layer F.Cu) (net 7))
 (segment (start 194.2 126) (end 194.57328 126.37328) (width 0.4) (layer F.Cu) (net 7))
 (segment (start 189.2248 123.9806) (end 193.3806 123.9806) (width 0.4) (layer F.Cu) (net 7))
 (segment (start 194.17308 124.77308) (end 194.2 124.77308) (width 0.4) (layer F.Cu) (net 7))
 (segment (start 194.2 124.77308) (end 198.826 124.77308) (width 0.4) (layer F.Cu) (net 7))
 (segment (start 193.3806 123.9806) (end 194.17308 124.77308) (width 0.4) (layer F.Cu) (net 7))
 (segment (start 208.8 129.4475) (end 208.8 126.5525) (width 0.4) (layer F.Cu) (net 7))
 (segment (start 198.2 117.8475) (end 198.2 113.2475) (width 0.4) (layer F.Cu) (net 7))
 (segment (start 198.2 113.2475) (end 198.1525 113.2) (width 0.4) (layer F.Cu) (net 7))
 (segment (start 195.5525 118.6) (end 196.4 118.6) (width 0.4) (layer F.Cu) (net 7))
 (segment (start 197.1525 117.8475) (end 198.2 117.8475) (width 0.4) (layer F.Cu) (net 7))
 (segment (start 196.4 118.6) (end 197.1525 117.8475) (width 0.4) (layer F.Cu) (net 7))
 (segment (start 188.2 149.2475) (end 188.2 146.72) (width 0.4) (layer F.Cu) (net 37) (status C00000))
 (segment (start 188.2 146.72) (end 188.25 146.67) (width 0.4) (layer F.Cu) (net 37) (status C00000))
 (segment (start 198.4 149.2475) (end 198.4 146.68) (width 0.4) (layer F.Cu) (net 32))
 (segment (start 198.4 146.68) (end 198.41 146.67) (width 0.4) (layer F.Cu) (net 32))
 (segment (start 201 149.2475) (end 201 146.72) (width 0.4) (layer F.Cu) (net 30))
 (segment (start 201 146.72) (end 200.95 146.67) (width 0.4) (layer F.Cu) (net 30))
 (segment (start 188.25 144.13) (end 188.25 141.2025) (width 0.4) (layer F.Cu) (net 36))
 (segment (start 188.25 141.2025) (end 188.2 141.1525) (width 0.4) (layer F.Cu) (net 36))
 (segment (start 190.79 144.13) (end 190.79 141.1625) (width 0.4) (layer F.Cu) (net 35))
 (segment (start 190.79 141.1625) (end 190.8 141.1525) (width 0.4) (layer F.Cu) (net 35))
 (segment (start 193.33 144.13) (end 193.33 141.2225) (width 0.4) (layer F.Cu) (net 34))
 (segment (start 193.33 141.2225) (end 193.4 141.1525) (width 0.4) (layer F.Cu) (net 34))
 (segment (start 198.41 144.13) (end 198.41 141.1625) (width 0.4) (layer F.Cu) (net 31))
 (segment (start 198.41 141.1625) (end 198.4 141.1525) (width 0.4) (layer F.Cu) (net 31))
 (segment (start 200.95 144.13) (end 200.95 141.2025) (width 0.4) (layer F.Cu) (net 29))
 (segment (start 200.95 141.2025) (end 201 141.1525) (width 0.4) (layer F.Cu) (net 29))
 (segment (start 193.20244 109.94828) (end 193.20244 111.39756) (width 0.4) (layer F.Cu) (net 38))
 (segment (start 191.4 113.2) (end 190.3525 113.2) (width 0.4) (layer F.Cu) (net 38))
 (segment (start 193.20244 111.39756) (end 191.4 113.2) (width 0.4) (layer F.Cu) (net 38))
 (segment (start 192.82398 121.98416) (end 192.82398 120.37602) (width 0.4) (layer F.Cu) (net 3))
 (segment (start 193.4 118.8475) (end 193.6475 118.6) (width 0.4) (layer F.Cu) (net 3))
 (segment (start 193.4 119.6) (end 193.4 118.8475) (width 0.4) (layer F.Cu) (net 3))
 (segment (start 192.8 120.2) (end 193.4 119.6) (width 0.4) (layer F.Cu) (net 3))
 (segment (start 192.8 120.35204) (end 192.8 120.2) (width 0.4) (layer F.Cu) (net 3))
 (segment (start 192.82398 120.37602) (end 192.8 120.35204) (width 0.4) (layer F.Cu) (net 3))
 (segment (start 201.8 124.9525) (end 204 124.9525) (width 0.4) (layer F.Cu) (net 14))
 (segment (start 198.826 125.57572) (end 201.17678 125.57572) (width 0.4) (layer F.Cu) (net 14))
 (segment (start 201.17678 125.57572) (end 201.8 124.9525) (width 0.4) (layer F.Cu) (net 14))
 (segment (start 192.8 114.0475) (end 192.8 113.2) (width 0.4) (layer F.Cu) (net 25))
 (segment (start 194 112) (end 194 109.94828) (width 0.4) (layer F.Cu) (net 25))
 (segment (start 192.8 113.2) (end 194 112) (width 0.4) (layer F.Cu) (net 25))
 (segment (start 194.79756 109.94828) (end 194.79756 114.00244) (width 0.4) (layer F.Cu) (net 26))
 (segment (start 190.8 115.6) (end 190.8 116.8475) (width 0.4) (layer F.Cu) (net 26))
 (segment (start 191.4 115) (end 190.8 115.6) (width 0.4) (layer F.Cu) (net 26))
 (segment (start 193.8 115) (end 191.4 115) (width 0.4) (layer F.Cu) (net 26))
 (segment (start 194.79756 114.00244) (end 193.8 115) (width 0.4) (layer F.Cu) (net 26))
 (segment (start 198.826 128.77612) (end 200.92862 128.77612) (width 0.4) (layer F.Cu) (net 5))
 (segment (start 200.92862 128.77612) (end 201.8 129.6475) (width 0.4) (layer F.Cu) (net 5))
 (segment (start 195 120.2) (end 195.4 119.8) (width 0.4) (layer F.Cu) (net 5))
 (segment (start 198.1525 119.8) (end 198.2 119.7525) (width 0.4) (layer F.Cu) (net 5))
 (segment (start 195.4 119.8) (end 198.1525 119.8) (width 0.4) (layer F.Cu) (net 5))
 (segment (start 194.42418 121.98416) (end 194.42418 120.77582) (width 0.4) (layer F.Cu) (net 5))
 (segment (start 195.2 121.95988) (end 195.22428 121.98416) (width 0.4) (layer F.Cu) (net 5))
 (segment (start 195.2 120.4) (end 195.2 121.95988) (width 0.4) (layer F.Cu) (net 5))
 (segment (start 195 120.2) (end 195.2 120.4) (width 0.4) (layer F.Cu) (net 5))
 (segment (start 194.42418 120.77582) (end 195 120.2) (width 0.4) (layer F.Cu) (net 5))
 (segment (start 196.2475 113.2) (end 196.2475 113.0475) (width 0.4) (layer F.Cu) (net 5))
 (segment (start 195.59766 112.39766) (end 195.59766 109.94828) (width 0.4) (layer F.Cu) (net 5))
 (segment (start 196.2475 113.0475) (end 195.59766 112.39766) (width 0.4) (layer F.Cu) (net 5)))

